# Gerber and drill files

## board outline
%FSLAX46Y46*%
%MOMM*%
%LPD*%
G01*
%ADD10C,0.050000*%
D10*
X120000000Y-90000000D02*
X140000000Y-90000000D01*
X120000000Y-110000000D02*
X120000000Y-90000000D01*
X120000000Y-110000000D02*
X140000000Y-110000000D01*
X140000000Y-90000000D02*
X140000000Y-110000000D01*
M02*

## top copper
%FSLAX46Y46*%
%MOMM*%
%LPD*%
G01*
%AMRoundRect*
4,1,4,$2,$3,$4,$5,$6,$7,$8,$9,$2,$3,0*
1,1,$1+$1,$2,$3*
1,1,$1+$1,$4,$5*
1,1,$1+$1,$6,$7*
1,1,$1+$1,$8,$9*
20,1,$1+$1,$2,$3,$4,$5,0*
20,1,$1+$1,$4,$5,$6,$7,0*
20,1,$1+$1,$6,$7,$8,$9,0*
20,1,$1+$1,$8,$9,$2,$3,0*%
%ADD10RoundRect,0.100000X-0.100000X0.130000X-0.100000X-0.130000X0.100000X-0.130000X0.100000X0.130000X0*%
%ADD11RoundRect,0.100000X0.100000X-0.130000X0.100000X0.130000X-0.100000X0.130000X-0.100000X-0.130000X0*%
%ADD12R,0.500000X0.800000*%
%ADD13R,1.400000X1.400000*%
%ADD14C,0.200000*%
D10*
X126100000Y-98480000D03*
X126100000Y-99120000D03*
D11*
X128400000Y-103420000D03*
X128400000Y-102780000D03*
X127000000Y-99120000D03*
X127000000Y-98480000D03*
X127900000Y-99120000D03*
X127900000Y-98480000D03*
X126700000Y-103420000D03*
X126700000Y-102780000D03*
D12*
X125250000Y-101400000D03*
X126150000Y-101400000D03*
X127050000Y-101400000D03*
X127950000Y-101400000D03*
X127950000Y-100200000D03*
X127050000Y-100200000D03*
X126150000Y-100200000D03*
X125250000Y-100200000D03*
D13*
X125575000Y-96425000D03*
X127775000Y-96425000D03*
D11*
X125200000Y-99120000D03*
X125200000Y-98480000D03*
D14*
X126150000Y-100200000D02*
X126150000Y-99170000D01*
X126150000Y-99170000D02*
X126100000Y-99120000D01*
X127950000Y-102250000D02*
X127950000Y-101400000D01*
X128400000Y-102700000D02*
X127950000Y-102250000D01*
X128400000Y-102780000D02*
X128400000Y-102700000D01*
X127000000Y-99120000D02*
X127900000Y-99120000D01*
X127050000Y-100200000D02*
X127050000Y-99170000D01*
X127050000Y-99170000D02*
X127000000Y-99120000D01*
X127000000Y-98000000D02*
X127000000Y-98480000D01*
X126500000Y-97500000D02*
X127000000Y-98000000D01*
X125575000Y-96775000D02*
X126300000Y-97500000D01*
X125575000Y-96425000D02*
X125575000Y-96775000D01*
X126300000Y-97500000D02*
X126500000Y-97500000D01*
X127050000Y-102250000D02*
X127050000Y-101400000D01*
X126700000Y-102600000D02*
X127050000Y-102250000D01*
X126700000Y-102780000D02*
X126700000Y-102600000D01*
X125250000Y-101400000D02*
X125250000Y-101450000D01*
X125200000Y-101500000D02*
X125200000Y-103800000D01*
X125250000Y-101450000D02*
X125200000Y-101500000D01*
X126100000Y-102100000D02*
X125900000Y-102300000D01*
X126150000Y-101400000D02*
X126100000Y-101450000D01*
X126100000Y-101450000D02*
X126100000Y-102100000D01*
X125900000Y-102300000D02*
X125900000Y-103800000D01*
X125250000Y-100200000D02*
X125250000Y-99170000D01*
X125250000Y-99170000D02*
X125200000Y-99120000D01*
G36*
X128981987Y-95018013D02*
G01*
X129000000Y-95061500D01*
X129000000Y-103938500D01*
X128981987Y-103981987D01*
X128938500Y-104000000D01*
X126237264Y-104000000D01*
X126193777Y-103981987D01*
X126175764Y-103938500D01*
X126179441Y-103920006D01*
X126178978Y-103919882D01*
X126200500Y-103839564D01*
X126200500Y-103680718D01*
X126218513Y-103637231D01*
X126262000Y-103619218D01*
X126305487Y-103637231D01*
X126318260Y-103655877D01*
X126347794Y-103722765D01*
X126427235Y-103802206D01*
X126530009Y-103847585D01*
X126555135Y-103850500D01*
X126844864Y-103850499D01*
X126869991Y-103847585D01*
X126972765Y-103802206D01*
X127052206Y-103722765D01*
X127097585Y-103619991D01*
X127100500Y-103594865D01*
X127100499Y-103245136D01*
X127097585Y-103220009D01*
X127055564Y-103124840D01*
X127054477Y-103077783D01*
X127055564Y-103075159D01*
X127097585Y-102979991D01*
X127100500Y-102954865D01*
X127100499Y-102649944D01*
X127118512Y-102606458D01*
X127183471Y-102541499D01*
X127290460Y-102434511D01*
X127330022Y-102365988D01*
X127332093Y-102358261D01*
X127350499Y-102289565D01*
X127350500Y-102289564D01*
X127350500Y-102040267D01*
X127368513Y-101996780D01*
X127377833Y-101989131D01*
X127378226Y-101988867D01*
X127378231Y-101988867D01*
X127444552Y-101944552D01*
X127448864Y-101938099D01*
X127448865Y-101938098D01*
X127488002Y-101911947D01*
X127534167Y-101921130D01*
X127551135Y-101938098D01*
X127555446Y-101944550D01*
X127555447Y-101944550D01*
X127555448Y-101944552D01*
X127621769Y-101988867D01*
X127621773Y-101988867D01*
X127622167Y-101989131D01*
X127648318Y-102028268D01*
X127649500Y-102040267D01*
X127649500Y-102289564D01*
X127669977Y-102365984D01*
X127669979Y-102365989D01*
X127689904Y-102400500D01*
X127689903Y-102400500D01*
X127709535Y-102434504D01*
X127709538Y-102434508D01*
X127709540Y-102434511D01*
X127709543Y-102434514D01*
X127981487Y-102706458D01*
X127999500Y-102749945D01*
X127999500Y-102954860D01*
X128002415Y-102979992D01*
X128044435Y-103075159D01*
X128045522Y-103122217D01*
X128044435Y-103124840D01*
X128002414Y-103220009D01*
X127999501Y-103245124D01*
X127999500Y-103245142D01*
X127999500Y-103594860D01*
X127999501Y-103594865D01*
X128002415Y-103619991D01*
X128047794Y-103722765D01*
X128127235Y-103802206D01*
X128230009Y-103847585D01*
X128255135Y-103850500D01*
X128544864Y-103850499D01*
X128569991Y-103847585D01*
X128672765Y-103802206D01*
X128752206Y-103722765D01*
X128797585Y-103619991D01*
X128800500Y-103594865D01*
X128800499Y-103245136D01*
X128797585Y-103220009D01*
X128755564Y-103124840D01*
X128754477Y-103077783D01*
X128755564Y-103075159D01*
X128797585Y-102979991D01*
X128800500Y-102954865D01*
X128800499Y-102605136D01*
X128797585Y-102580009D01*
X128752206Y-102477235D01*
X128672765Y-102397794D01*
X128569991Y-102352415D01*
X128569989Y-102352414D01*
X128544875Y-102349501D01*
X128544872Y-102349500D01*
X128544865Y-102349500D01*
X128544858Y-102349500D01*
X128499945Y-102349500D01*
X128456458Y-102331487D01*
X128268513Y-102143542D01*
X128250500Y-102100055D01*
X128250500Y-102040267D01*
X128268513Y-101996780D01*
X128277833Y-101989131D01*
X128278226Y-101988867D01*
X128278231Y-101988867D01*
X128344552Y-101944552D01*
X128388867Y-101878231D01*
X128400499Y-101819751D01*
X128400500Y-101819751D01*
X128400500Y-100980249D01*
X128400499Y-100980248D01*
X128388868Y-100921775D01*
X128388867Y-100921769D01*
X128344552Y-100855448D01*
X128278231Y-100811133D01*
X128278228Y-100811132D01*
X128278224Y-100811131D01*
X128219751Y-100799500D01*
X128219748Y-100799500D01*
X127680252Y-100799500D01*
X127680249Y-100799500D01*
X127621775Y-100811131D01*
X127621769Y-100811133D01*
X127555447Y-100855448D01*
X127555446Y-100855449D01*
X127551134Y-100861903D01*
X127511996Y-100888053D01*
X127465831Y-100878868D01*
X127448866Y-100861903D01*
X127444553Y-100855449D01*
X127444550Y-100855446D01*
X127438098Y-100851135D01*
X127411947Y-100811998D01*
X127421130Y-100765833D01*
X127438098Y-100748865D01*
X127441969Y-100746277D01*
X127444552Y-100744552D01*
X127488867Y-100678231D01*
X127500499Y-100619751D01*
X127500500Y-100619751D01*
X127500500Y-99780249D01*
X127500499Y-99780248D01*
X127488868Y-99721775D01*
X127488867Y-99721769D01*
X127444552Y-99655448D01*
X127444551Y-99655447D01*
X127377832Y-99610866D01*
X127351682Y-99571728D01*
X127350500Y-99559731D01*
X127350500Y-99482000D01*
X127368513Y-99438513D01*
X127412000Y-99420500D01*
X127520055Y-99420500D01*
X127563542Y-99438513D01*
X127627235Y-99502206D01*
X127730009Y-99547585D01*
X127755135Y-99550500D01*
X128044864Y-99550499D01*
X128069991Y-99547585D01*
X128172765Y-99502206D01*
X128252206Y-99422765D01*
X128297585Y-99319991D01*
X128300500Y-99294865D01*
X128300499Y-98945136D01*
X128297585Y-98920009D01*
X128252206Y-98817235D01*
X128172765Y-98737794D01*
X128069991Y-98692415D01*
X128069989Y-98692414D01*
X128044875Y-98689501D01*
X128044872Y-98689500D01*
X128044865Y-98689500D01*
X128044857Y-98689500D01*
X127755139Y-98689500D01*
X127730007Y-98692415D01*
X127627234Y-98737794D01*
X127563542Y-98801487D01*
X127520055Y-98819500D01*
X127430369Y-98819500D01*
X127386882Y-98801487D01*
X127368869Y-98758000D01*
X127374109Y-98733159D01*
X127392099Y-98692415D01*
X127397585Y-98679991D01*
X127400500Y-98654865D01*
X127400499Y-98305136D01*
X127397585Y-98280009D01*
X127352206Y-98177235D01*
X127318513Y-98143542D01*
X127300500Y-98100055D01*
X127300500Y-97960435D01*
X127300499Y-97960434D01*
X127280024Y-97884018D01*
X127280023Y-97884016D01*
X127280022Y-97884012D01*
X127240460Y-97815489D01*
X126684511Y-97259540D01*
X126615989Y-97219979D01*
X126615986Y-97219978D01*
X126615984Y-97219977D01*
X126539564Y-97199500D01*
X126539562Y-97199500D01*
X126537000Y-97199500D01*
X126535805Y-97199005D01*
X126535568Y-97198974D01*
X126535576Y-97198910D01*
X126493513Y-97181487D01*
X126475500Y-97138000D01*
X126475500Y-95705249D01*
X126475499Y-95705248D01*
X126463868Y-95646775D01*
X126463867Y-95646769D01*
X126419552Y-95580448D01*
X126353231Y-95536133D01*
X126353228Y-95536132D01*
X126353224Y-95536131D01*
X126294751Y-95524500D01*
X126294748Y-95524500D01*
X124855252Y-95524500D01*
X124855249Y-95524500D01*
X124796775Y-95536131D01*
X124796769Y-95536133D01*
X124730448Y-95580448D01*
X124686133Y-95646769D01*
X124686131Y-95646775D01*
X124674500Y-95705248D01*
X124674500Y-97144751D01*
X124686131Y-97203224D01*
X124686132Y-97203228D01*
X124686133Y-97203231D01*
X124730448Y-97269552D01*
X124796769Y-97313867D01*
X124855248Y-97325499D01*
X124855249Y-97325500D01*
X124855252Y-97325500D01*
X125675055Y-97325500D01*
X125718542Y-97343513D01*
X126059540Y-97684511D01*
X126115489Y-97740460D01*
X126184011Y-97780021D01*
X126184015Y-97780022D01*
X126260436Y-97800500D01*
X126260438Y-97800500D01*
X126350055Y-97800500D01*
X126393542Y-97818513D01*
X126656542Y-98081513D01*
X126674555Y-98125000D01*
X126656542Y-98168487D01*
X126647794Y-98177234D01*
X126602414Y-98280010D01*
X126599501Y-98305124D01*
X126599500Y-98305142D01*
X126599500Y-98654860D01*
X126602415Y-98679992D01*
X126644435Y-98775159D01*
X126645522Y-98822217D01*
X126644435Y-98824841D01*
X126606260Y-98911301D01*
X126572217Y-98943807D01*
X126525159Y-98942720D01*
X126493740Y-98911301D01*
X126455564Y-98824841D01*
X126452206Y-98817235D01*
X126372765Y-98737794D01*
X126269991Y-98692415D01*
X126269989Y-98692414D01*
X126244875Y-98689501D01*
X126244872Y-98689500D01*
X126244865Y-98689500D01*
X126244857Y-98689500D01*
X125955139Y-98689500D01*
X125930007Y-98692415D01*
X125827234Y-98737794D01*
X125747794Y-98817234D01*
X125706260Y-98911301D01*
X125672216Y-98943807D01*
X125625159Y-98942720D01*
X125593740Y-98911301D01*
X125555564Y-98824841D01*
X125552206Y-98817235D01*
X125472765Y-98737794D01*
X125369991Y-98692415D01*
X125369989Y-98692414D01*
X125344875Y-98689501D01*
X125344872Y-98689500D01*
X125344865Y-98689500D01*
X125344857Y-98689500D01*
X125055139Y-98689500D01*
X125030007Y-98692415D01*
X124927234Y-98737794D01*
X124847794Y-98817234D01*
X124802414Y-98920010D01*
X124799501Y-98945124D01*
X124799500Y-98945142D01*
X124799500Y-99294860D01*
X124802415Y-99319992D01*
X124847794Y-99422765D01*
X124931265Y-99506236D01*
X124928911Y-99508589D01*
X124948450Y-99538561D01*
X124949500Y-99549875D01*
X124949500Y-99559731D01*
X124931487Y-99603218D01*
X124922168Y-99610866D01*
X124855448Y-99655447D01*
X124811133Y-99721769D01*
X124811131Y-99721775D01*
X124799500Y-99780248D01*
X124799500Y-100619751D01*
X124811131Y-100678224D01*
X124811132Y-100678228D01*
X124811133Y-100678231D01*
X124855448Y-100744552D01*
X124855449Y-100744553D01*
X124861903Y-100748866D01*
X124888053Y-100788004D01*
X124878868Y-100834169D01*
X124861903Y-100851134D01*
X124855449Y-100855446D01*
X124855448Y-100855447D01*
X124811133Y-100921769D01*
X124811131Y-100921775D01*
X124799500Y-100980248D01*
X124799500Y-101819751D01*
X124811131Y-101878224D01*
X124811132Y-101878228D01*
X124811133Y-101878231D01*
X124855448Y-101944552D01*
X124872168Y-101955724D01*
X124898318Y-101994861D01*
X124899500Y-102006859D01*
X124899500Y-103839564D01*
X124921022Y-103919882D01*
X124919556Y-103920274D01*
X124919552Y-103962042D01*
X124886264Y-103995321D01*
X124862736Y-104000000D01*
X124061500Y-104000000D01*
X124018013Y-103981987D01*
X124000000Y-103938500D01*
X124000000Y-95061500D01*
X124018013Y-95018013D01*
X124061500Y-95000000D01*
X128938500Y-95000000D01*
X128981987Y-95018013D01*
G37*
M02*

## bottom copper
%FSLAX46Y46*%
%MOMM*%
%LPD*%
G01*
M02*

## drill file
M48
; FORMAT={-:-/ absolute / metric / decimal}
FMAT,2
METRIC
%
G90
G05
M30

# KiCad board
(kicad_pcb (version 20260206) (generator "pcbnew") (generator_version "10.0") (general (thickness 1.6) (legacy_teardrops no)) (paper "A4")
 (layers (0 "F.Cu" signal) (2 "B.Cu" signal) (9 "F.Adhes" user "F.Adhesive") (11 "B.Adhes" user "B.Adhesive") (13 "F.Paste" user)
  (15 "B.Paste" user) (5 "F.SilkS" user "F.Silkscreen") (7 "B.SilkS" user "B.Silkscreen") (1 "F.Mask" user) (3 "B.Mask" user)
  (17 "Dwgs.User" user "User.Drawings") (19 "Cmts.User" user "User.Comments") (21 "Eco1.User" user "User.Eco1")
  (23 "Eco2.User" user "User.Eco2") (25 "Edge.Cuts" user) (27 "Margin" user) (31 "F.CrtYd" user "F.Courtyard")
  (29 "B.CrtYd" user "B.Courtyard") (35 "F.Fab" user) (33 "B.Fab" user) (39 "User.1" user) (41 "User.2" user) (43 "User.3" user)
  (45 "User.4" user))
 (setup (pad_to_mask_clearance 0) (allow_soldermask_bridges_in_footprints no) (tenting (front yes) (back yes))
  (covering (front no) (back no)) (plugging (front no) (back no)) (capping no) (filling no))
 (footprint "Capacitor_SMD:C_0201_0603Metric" (layer "F.Cu") (at 126.1 98.8 -90)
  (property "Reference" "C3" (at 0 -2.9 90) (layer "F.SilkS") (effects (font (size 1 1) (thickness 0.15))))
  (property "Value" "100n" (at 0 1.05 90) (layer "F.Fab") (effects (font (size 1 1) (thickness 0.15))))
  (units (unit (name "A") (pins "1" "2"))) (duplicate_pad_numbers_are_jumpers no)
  (pad "" smd roundrect (at -0.345 0 270) (size 0.318 0.36) (layers "F.Paste") (roundrect_rratio 0.25))
  (pad "" smd roundrect (at 0.345 0 270) (size 0.318 0.36) (layers "F.Paste") (roundrect_rratio 0.25))
  (pad "1" smd roundrect (at -0.32 0 270) (size 0.46 0.4) (layers "F.Cu" "F.Mask") (roundrect_rratio 0.25) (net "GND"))
  (pad "2" smd roundrect (at 0.32 0 270) (size 0.46 0.4) (layers "F.Cu" "F.Mask") (roundrect_rratio 0.25) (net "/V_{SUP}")))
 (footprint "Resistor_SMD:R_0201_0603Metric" (layer "F.Cu") (at 128.4 103.1 90)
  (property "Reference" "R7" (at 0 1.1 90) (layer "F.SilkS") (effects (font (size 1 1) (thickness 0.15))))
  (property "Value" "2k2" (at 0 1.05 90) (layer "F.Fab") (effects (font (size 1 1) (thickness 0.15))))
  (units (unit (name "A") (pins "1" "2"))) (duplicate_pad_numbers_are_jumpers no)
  (pad "" smd roundrect (at -0.345 0 90) (size 0.318 0.36) (layers "F.Paste") (roundrect_rratio 0.25))
  (pad "" smd roundrect (at 0.345 0 90) (size 0.318 0.36) (layers "F.Paste") (roundrect_rratio 0.25))
  (pad "1" smd roundrect (at -0.32 0 90) (size 0.46 0.4) (layers "F.Cu" "F.Mask") (roundrect_rratio 0.25) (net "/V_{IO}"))
  (pad "2" smd roundrect (at 0.32 0 90) (size 0.46 0.4) (layers "F.Cu" "F.Mask") (roundrect_rratio 0.25) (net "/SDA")))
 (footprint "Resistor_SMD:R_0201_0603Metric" (layer "F.Cu") (at 127 98.8 90)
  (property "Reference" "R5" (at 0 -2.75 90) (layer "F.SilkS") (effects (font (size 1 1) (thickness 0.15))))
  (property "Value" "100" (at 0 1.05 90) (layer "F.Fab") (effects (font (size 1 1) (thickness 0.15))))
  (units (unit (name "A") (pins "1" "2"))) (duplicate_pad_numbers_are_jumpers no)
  (pad "" smd roundrect (at -0.345 0 90) (size 0.318 0.36) (layers "F.Paste") (roundrect_rratio 0.25))
  (pad "" smd roundrect (at 0.345 0 90) (size 0.318 0.36) (layers "F.Paste") (roundrect_rratio 0.25))
  (pad "1" smd roundrect (at -0.32 0 90) (size 0.46 0.4) (layers "F.Cu" "F.Mask") (roundrect_rratio 0.25) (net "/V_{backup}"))
  (pad "2" smd roundrect (at 0.32 0 90) (size 0.46 0.4) (layers "F.Cu" "F.Mask") (roundrect_rratio 0.25) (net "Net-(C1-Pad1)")))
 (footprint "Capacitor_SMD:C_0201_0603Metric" (layer "F.Cu") (at 127.9 98.8 90)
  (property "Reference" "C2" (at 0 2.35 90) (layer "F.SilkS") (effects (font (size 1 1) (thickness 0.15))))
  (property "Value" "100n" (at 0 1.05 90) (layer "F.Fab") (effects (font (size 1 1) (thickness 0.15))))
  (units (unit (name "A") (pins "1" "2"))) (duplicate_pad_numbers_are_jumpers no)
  (pad "" smd roundrect (at -0.345 0 90) (size 0.318 0.36) (layers "F.Paste") (roundrect_rratio 0.25))
  (pad "" smd roundrect (at 0.345 0 90) (size 0.318 0.36) (layers "F.Paste") (roundrect_rratio 0.25))
  (pad "1" smd roundrect (at -0.32 0 90) (size 0.46 0.4) (layers "F.Cu" "F.Mask") (roundrect_rratio 0.25) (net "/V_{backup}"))
  (pad "2" smd roundrect (at 0.32 0 90) (size 0.46 0.4) (layers "F.Cu" "F.Mask") (roundrect_rratio 0.25) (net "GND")))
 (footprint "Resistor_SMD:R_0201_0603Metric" (layer "F.Cu") (at 126.7 103.1 90)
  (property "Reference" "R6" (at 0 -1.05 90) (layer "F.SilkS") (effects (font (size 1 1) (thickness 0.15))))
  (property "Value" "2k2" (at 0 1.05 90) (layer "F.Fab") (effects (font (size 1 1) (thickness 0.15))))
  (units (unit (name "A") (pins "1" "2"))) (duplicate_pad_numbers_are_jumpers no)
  (pad "" smd roundrect (at -0.345 0 90) (size 0.318 0.36) (layers "F.Paste") (roundrect_rratio 0.25))
  (pad "" smd roundrect (at 0.345 0 90) (size 0.318 0.36) (layers "F.Paste") (roundrect_rratio 0.25))
  (pad "1" smd roundrect (at -0.32 0 90) (size 0.46 0.4) (layers "F.Cu" "F.Mask") (roundrect_rratio 0.25) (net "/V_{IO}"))
  (pad "2" smd roundrect (at 0.32 0 90) (size 0.46 0.4) (layers "F.Cu" "F.Mask") (roundrect_rratio 0.25) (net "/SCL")))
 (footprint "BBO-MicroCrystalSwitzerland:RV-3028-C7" (layer "F.Cu") (at 126.6 100.8)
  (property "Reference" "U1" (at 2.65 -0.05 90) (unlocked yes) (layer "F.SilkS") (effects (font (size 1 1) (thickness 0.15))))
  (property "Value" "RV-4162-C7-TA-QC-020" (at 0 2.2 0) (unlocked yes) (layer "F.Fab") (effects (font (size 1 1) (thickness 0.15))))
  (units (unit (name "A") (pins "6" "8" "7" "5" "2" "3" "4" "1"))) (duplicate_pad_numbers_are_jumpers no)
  (pad "1" smd rect (at -1.35 0.6) (size 0.5 0.8) (layers "F.Cu" "F.Mask" "F.Paste") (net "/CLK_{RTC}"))
  (pad "2" smd rect (at -0.45 0.6) (size 0.5 0.8) (layers "F.Cu" "F.Mask" "F.Paste") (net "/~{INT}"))
  (pad "3" smd rect (at 0.45 0.6) (size 0.5 0.8) (layers "F.Cu" "F.Mask" "F.Paste") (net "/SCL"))
  (pad "4" smd rect (at 1.35 0.6) (size 0.5 0.8) (layers "F.Cu" "F.Mask" "F.Paste") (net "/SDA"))
  (pad "5" smd rect (at 1.35 -0.6) (size 0.5 0.8) (layers "F.Cu" "F.Mask" "F.Paste") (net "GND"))
  (pad "6" smd rect (at 0.45 -0.6) (size 0.5 0.8) (layers "F.Cu" "F.Mask" "F.Paste") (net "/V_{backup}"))
  (pad "7" smd rect (at -0.45 -0.6) (size 0.5 0.8) (layers "F.Cu" "F.Mask" "F.Paste") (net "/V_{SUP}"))
  (pad "8" smd rect (at -1.35 -0.6) (size 0.5 0.8) (layers "F.Cu" "F.Mask" "F.Paste") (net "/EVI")))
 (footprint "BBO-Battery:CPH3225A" (layer "F.Cu") (at 126.675 96.425)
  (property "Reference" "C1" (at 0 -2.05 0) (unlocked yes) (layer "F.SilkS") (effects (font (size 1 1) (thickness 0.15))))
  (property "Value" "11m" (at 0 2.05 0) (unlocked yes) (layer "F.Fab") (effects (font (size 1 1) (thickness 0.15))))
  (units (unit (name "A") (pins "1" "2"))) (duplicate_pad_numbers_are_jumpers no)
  (pad "1" smd rect (at -1.1 0) (size 1.4 1.4) (layers "F.Cu" "F.Mask" "F.Paste") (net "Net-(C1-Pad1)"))
  (pad "2" smd rect (at 1.1 0) (size 1.4 1.4) (layers "F.Cu" "F.Mask" "F.Paste") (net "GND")))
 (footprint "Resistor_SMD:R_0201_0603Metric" (layer "F.Cu") (at 125.2 98.8 90)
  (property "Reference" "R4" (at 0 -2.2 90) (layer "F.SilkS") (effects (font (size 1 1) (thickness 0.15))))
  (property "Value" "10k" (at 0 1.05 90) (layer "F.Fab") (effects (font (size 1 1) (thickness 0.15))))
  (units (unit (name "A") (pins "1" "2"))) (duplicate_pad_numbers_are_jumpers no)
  (pad "" smd roundrect (at -0.345 0 90) (size 0.318 0.36) (layers "F.Paste") (roundrect_rratio 0.25))
  (pad "" smd roundrect (at 0.345 0 90) (size 0.318 0.36) (layers "F.Paste") (roundrect_rratio 0.25))
  (pad "1" smd roundrect (at -0.32 0 90) (size 0.46 0.4) (layers "F.Cu" "F.Mask") (roundrect_rratio 0.25) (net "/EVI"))
  (pad "2" smd roundrect (at 0.32 0 90) (size 0.46 0.4) (layers "F.Cu" "F.Mask") (roundrect_rratio 0.25) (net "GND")))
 (gr_line (start 120 90) (end 140 90) (stroke (width 0.05) (type default)) (layer "Edge.Cuts"))
 (gr_line (start 120 110) (end 120 90) (stroke (width 0.05) (type default)) (layer "Edge.Cuts"))
 (gr_line (start 120 110) (end 140 110) (stroke (width 0.05) (type default)) (layer "Edge.Cuts"))
 (gr_line (start 140 90) (end 140 110) (stroke (width 0.05) (type default)) (layer "Edge.Cuts"))
 (segment (start 126.15 100.2) (end 126.15 99.17) (width 0.2) (layer "F.Cu") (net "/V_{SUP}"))
 (segment (start 126.15 99.17) (end 126.1 99.12) (width 0.2) (layer "F.Cu") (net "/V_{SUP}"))
 (segment (start 127.95 102.25) (end 127.95 101.4) (width 0.2) (layer "F.Cu") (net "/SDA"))
 (segment (start 128.4 102.7) (end 127.95 102.25) (width 0.2) (layer "F.Cu") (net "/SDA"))
 (segment (start 128.4 102.78) (end 128.4 102.7) (width 0.2) (layer "F.Cu") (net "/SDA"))
 (segment (start 127 99.12) (end 127.9 99.12) (width 0.2) (layer "F.Cu") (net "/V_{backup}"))
 (segment (start 127.05 100.2) (end 127.05 99.17) (width 0.2) (layer "F.Cu") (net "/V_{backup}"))
 (segment (start 127.05 99.17) (end 127 99.12) (width 0.2) (layer "F.Cu") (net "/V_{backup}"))
 (segment (start 127 98) (end 127 98.48) (width 0.2) (layer "F.Cu") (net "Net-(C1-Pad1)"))
 (segment (start 126.5 97.5) (end 127 98) (width 0.2) (layer "F.Cu") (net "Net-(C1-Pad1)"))
 (segment (start 125.575 96.775) (end 126.3 97.5) (width 0.2) (layer "F.Cu") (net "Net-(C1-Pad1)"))
 (segment (start 125.575 96.425) (end 125.575 96.775) (width 0.2) (layer "F.Cu") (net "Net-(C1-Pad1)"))
 (segment (start 126.3 97.5) (end 126.5 97.5) (width 0.2) (layer "F.Cu") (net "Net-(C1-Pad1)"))
 (segment (start 127.05 102.25) (end 127.05 101.4) (width 0.2) (layer "F.Cu") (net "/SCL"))
 (segment (start 126.7 102.6) (end 127.05 102.25) (width 0.2) (layer "F.Cu") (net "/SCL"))
 (segment (start 126.7 102.78) (end 126.7 102.6) (width 0.2) (layer "F.Cu") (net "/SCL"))
 (segment (start 125.25 101.4) (end 125.25 101.45) (width 0.2) (layer "F.Cu") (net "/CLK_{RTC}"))
 (segment (start 125.2 101.5) (end 125.2 103.8) (width 0.2) (layer "F.Cu") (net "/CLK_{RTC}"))
 (segment (start 125.25 101.45) (end 125.2 101.5) (width 0.2) (layer "F.Cu") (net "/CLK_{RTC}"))
 (segment (start 126.1 102.1) (end 125.9 102.3) (width 0.2) (layer "F.Cu") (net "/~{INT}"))
 (segment (start 126.15 101.4) (end 126.1 101.45) (width 0.2) (layer "F.Cu") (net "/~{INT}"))
 (segment (start 126.1 101.45) (end 126.1 102.1) (width 0.2) (layer "F.Cu") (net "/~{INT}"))
 (segment (start 125.9 102.3) (end 125.9 103.8) (width 0.2) (layer "F.Cu") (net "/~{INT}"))
 (segment (start 125.25 100.2) (end 125.25 99.17) (width 0.2) (layer "F.Cu") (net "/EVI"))
 (segment (start 125.25 99.17) (end 125.2 99.12) (width 0.2) (layer "F.Cu") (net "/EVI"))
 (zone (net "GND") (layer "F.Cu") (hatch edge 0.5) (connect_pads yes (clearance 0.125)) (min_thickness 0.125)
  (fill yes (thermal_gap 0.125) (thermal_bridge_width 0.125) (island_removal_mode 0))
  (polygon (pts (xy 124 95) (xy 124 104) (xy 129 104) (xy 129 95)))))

